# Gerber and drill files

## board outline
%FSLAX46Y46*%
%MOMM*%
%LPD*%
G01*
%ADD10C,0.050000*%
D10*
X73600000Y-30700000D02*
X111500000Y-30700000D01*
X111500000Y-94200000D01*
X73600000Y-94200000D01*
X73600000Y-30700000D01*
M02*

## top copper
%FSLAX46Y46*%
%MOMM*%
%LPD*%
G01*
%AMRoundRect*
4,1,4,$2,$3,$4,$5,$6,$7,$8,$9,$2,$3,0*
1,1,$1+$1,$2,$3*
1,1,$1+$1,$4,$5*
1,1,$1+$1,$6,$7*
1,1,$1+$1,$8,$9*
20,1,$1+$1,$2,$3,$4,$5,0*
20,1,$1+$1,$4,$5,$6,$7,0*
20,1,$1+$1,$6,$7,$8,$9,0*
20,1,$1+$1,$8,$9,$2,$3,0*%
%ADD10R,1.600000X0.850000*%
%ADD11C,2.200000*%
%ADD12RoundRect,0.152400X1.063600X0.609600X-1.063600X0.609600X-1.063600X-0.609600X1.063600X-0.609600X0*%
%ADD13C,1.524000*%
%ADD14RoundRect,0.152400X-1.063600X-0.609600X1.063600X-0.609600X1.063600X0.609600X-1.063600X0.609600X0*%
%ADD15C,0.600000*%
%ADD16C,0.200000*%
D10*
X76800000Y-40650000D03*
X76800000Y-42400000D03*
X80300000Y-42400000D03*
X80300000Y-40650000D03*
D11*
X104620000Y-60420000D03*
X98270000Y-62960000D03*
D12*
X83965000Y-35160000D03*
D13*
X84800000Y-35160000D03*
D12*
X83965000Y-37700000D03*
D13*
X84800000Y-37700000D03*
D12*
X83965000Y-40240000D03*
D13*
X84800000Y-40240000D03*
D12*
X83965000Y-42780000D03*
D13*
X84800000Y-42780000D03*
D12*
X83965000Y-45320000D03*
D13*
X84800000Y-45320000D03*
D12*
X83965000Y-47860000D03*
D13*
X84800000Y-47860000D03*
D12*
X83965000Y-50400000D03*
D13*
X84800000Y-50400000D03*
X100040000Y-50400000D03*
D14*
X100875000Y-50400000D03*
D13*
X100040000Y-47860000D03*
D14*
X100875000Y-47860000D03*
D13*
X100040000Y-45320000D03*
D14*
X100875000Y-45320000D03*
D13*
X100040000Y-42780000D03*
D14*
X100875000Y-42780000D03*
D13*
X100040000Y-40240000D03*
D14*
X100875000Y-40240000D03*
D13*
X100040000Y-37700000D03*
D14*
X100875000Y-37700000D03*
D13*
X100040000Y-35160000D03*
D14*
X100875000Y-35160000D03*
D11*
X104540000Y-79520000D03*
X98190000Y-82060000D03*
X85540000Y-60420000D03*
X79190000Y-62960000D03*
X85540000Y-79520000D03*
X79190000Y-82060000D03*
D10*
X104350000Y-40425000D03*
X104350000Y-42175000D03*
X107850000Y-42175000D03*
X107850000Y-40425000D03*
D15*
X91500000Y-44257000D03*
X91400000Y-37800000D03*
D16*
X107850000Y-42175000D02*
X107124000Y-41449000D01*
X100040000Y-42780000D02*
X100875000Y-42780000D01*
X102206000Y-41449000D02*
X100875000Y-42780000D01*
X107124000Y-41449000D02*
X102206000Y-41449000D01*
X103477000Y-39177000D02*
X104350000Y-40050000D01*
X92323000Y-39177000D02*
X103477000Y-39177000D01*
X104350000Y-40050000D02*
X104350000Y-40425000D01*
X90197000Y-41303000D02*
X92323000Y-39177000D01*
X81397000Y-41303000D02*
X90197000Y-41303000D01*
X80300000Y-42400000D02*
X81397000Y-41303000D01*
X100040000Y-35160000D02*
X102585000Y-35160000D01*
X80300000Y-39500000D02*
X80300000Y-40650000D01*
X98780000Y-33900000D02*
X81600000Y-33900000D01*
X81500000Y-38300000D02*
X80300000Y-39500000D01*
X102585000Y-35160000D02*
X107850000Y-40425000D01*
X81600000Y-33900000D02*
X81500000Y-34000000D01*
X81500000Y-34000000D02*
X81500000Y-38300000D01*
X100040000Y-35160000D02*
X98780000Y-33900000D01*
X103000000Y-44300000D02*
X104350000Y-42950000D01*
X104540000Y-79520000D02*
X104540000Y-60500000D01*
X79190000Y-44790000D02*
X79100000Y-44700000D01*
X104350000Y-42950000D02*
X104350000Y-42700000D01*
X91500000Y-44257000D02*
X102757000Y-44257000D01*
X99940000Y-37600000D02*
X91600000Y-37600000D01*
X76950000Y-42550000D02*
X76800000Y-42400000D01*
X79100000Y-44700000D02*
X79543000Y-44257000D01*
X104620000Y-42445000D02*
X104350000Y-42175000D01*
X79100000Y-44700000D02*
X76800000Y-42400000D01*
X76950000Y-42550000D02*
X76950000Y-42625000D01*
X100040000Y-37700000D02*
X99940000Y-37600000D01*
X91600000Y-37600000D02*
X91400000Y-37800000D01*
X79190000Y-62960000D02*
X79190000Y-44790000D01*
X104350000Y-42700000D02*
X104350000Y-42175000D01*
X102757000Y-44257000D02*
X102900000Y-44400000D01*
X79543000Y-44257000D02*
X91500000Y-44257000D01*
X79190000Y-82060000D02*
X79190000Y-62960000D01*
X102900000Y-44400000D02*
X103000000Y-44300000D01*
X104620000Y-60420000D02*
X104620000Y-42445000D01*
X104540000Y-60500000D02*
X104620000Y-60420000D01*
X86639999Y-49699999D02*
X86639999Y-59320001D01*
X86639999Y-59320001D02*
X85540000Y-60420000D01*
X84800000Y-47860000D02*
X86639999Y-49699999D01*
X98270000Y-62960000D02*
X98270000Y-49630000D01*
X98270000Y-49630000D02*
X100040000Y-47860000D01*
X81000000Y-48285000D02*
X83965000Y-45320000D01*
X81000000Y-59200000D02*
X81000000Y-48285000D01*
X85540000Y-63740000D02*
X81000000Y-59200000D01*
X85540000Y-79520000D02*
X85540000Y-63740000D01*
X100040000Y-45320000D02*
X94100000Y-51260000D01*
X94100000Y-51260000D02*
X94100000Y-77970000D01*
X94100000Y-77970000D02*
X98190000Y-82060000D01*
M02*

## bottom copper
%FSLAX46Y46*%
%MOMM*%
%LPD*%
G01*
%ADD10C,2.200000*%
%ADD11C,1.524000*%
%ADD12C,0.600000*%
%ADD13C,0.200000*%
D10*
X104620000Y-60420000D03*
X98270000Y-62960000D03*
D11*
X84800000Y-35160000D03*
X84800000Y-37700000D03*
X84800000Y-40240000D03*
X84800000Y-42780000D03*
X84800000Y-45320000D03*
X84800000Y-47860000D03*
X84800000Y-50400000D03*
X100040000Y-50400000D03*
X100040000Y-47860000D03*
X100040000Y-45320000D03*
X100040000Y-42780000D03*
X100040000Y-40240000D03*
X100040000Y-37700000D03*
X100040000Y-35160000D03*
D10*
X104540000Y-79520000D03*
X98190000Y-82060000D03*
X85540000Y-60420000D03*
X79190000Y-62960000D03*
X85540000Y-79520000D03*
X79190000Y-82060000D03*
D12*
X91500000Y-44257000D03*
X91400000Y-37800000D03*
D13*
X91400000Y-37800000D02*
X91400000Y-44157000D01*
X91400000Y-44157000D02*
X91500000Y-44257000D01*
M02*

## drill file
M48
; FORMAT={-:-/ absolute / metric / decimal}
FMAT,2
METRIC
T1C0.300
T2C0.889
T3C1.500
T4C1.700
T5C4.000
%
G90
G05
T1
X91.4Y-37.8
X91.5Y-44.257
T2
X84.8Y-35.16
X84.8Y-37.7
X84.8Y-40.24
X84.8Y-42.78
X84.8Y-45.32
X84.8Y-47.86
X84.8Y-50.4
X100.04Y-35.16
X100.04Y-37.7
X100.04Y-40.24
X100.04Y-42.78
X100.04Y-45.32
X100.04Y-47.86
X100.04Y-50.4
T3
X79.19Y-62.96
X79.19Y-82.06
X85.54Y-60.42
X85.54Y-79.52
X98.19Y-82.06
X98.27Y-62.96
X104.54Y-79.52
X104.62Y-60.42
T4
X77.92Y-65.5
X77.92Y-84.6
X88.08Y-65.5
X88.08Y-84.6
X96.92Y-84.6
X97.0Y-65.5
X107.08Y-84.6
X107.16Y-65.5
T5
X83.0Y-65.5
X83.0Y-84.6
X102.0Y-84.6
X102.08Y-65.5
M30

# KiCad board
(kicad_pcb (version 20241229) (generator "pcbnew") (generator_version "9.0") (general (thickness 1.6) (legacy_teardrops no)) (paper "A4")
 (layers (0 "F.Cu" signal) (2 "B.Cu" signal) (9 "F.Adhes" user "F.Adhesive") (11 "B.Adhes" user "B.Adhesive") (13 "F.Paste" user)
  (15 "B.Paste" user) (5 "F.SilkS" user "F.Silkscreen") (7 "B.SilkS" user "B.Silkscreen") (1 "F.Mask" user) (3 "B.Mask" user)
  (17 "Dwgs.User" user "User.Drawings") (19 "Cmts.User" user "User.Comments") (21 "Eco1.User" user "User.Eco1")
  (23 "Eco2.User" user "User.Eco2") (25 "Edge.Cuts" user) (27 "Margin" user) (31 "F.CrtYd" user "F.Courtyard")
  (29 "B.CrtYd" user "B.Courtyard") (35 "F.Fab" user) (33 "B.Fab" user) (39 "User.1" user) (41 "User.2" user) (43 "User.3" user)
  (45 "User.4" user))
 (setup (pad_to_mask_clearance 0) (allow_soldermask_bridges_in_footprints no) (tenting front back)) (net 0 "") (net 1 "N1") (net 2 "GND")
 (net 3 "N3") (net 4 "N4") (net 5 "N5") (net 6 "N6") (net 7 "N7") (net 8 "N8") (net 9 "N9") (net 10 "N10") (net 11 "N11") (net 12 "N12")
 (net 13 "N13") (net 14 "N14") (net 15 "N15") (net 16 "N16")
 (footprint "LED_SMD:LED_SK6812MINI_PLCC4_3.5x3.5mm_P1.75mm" (layer "F.Cu") (at 78.55 41.525)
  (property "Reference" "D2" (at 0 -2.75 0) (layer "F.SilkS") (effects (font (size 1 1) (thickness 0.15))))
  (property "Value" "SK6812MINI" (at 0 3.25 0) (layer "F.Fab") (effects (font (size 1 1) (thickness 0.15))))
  (pad "1" smd rect (at -1.75 -0.875) (size 1.6 0.85) (layers "F.Cu" "F.Mask" "F.Paste") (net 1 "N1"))
  (pad "2" smd rect (at -1.75 0.875) (size 1.6 0.85) (layers "F.Cu" "F.Mask" "F.Paste") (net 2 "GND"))
  (pad "3" smd rect (at 1.75 0.875) (size 1.6 0.85) (layers "F.Cu" "F.Mask" "F.Paste") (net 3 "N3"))
  (pad "4" smd rect (at 1.75 -0.875) (size 1.6 0.85) (layers "F.Cu" "F.Mask" "F.Paste") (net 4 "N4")))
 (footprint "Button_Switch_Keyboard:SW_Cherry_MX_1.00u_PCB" (layer "F.Cu") (at 104.62 60.42)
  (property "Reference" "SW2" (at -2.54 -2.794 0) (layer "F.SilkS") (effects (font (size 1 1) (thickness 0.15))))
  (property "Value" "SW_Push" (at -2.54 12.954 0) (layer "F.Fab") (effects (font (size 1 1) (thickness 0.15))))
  (pad "" np_thru_hole circle (at -7.62 5.08) (size 1.7 1.7) (drill 1.7) (layers "*.Cu" "*.Mask"))
  (pad "" np_thru_hole circle (at -2.54 5.08) (size 4 4) (drill 4) (layers "*.Cu" "*.Mask"))
  (pad "" np_thru_hole circle (at 2.54 5.08) (size 1.7 1.7) (drill 1.7) (layers "*.Cu" "*.Mask"))
  (pad "1" thru_hole circle (at 0 0) (size 2.2 2.2) (drill 1.5) (layers "*.Cu" "*.Mask") (remove_unused_layers no) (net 2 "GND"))
  (pad "2" thru_hole circle (at -6.35 2.54) (size 2.2 2.2) (drill 1.5) (layers "*.Cu" "*.Mask") (remove_unused_layers no) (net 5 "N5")))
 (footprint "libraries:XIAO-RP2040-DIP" (layer "F.Cu") (at 92.42 42.78)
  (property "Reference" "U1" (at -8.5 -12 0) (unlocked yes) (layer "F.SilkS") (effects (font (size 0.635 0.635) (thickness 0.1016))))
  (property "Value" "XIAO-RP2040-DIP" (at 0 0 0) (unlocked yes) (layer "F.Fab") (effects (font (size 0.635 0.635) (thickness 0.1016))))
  (pad "1" smd roundrect (at -8.455 -7.62 180) (size 2.432 1.524) (layers "F.Cu" "F.Mask") (roundrect_rratio 0.1) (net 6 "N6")
   (thermal_bridge_angle 45))
  (pad "1" thru_hole circle (at -7.62 -7.62 180) (size 1.524 1.524) (drill 0.889) (layers "*.Cu" "*.Mask") (remove_unused_layers no)
   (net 6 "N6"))
  (pad "2" smd roundrect (at -8.455 -5.08 180) (size 2.432 1.524) (layers "F.Cu" "F.Mask") (roundrect_rratio 0.1) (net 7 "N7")
   (thermal_bridge_angle 45))
  (pad "2" thru_hole circle (at -7.62 -5.08 180) (size 1.524 1.524) (drill 0.889) (layers "*.Cu" "*.Mask") (remove_unused_layers no)
   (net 7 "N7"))
  (pad "3" smd roundrect (at -8.455 -2.54 180) (size 2.432 1.524) (layers "F.Cu" "F.Mask") (roundrect_rratio 0.1) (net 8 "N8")
   (thermal_bridge_angle 45))
  (pad "3" thru_hole circle (at -7.62 -2.54 180) (size 1.524 1.524) (drill 0.889) (layers "*.Cu" "*.Mask") (remove_unused_layers no)
   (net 8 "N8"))
  (pad "4" smd roundrect (at -8.455 0 180) (size 2.432 1.524) (layers "F.Cu" "F.Mask") (roundrect_rratio 0.1) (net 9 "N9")
   (thermal_bridge_angle 45))
  (pad "4" thru_hole circle (at -7.62 0 180) (size 1.524 1.524) (drill 0.889) (layers "*.Cu" "*.Mask") (remove_unused_layers no)
   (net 9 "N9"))
  (pad "5" smd roundrect (at -8.455 2.54 180) (size 2.432 1.524) (layers "F.Cu" "F.Mask") (roundrect_rratio 0.1) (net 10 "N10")
   (thermal_bridge_angle 45))
  (pad "5" thru_hole circle (at -7.62 2.54 180) (size 1.524 1.524) (drill 0.889) (layers "*.Cu" "*.Mask") (remove_unused_layers no)
   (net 10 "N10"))
  (pad "6" smd roundrect (at -8.455 5.08 180) (size 2.432 1.524) (layers "F.Cu" "F.Mask") (roundrect_rratio 0.1) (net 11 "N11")
   (thermal_bridge_angle 45))
  (pad "6" thru_hole circle (at -7.62 5.08 180) (size 1.524 1.524) (drill 0.889) (layers "*.Cu" "*.Mask") (remove_unused_layers no)
   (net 11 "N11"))
  (pad "7" smd roundrect (at -8.455 7.62 180) (size 2.432 1.524) (layers "F.Cu" "F.Mask") (roundrect_rratio 0.1) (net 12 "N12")
   (thermal_bridge_angle 45))
  (pad "7" thru_hole circle (at -7.62 7.62 180) (size 1.524 1.524) (drill 0.889) (layers "*.Cu" "*.Mask") (remove_unused_layers no)
   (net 12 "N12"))
  (pad "8" thru_hole circle (at 7.62 7.62) (size 1.524 1.524) (drill 0.889) (layers "*.Cu" "*.Mask") (remove_unused_layers no)
   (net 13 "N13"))
  (pad "8" smd roundrect (at 8.455 7.62) (size 2.432 1.524) (layers "F.Cu" "F.Mask") (roundrect_rratio 0.1) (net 13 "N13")
   (thermal_bridge_angle 45))
  (pad "9" thru_hole circle (at 7.62 5.08) (size 1.524 1.524) (drill 0.889) (layers "*.Cu" "*.Mask") (remove_unused_layers no) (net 5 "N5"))
  (pad "9" smd roundrect (at 8.455 5.08) (size 2.432 1.524) (layers "F.Cu" "F.Mask") (roundrect_rratio 0.1) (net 5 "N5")
   (thermal_bridge_angle 45))
  (pad "10" thru_hole circle (at 7.62 2.54) (size 1.524 1.524) (drill 0.889) (layers "*.Cu" "*.Mask") (remove_unused_layers no)
   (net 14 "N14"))
  (pad "10" smd roundrect (at 8.455 2.54) (size 2.432 1.524) (layers "F.Cu" "F.Mask") (roundrect_rratio 0.1) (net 14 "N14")
   (thermal_bridge_angle 45))
  (pad "11" thru_hole circle (at 7.62 0) (size 1.524 1.524) (drill 0.889) (layers "*.Cu" "*.Mask") (remove_unused_layers no) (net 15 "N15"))
  (pad "11" smd roundrect (at 8.455 0) (size 2.432 1.524) (layers "F.Cu" "F.Mask") (roundrect_rratio 0.1) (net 15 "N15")
   (thermal_bridge_angle 45))
  (pad "12" thru_hole circle (at 7.62 -2.54) (size 1.524 1.524) (drill 0.889) (layers "*.Cu" "*.Mask") (remove_unused_layers no)
   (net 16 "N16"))
  (pad "12" smd roundrect (at 8.455 -2.54) (size 2.432 1.524) (layers "F.Cu" "F.Mask") (roundrect_rratio 0.1) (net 16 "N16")
   (thermal_bridge_angle 45))
  (pad "13" thru_hole circle (at 7.62 -5.08) (size 1.524 1.524) (drill 0.889) (layers "*.Cu" "*.Mask") (remove_unused_layers no)
   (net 2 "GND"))
  (pad "13" smd roundrect (at 8.455 -5.08) (size 2.432 1.524) (layers "F.Cu" "F.Mask") (roundrect_rratio 0.1) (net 2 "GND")
   (thermal_bridge_angle 45))
  (pad "14" thru_hole circle (at 7.62 -7.62) (size 1.524 1.524) (drill 0.889) (layers "*.Cu" "*.Mask") (remove_unused_layers no)
   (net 4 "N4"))
  (pad "14" smd roundrect (at 8.455 -7.62) (size 2.432 1.524) (layers "F.Cu" "F.Mask") (roundrect_rratio 0.1) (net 4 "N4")
   (thermal_bridge_angle 45)))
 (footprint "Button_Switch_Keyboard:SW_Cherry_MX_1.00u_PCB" (layer "F.Cu") (at 104.54 79.52)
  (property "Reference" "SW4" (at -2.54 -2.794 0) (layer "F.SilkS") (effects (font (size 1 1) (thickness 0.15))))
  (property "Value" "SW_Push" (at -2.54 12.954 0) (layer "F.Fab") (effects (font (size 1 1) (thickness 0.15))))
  (pad "" np_thru_hole circle (at -7.62 5.08) (size 1.7 1.7) (drill 1.7) (layers "*.Cu" "*.Mask"))
  (pad "" np_thru_hole circle (at -2.54 5.08) (size 4 4) (drill 4) (layers "*.Cu" "*.Mask"))
  (pad "" np_thru_hole circle (at 2.54 5.08) (size 1.7 1.7) (drill 1.7) (layers "*.Cu" "*.Mask"))
  (pad "1" thru_hole circle (at 0 0) (size 2.2 2.2) (drill 1.5) (layers "*.Cu" "*.Mask") (remove_unused_layers no) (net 2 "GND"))
  (pad "2" thru_hole circle (at -6.35 2.54) (size 2.2 2.2) (drill 1.5) (layers "*.Cu" "*.Mask") (remove_unused_layers no) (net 14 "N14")))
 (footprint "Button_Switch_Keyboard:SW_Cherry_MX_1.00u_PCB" (layer "F.Cu") (at 85.54 60.42)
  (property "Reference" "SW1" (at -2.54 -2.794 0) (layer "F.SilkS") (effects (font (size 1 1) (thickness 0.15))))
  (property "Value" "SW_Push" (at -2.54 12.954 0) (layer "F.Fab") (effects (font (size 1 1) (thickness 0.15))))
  (pad "" np_thru_hole circle (at -7.62 5.08) (size 1.7 1.7) (drill 1.7) (layers "*.Cu" "*.Mask"))
  (pad "" np_thru_hole circle (at -2.54 5.08) (size 4 4) (drill 4) (layers "*.Cu" "*.Mask"))
  (pad "" np_thru_hole circle (at 2.54 5.08) (size 1.7 1.7) (drill 1.7) (layers "*.Cu" "*.Mask"))
  (pad "1" thru_hole circle (at 0 0) (size 2.2 2.2) (drill 1.5) (layers "*.Cu" "*.Mask") (remove_unused_layers no) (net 11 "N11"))
  (pad "2" thru_hole circle (at -6.35 2.54) (size 2.2 2.2) (drill 1.5) (layers "*.Cu" "*.Mask") (remove_unused_layers no) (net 2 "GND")))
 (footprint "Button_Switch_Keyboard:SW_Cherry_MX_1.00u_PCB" (layer "F.Cu") (at 85.54 79.52)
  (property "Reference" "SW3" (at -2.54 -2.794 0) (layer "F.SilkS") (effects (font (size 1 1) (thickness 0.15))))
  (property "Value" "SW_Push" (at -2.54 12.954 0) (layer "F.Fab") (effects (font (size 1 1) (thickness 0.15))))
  (pad "" np_thru_hole circle (at -7.62 5.08) (size 1.7 1.7) (drill 1.7) (layers "*.Cu" "*.Mask"))
  (pad "" np_thru_hole circle (at -2.54 5.08) (size 4 4) (drill 4) (layers "*.Cu" "*.Mask"))
  (pad "" np_thru_hole circle (at 2.54 5.08) (size 1.7 1.7) (drill 1.7) (layers "*.Cu" "*.Mask"))
  (pad "1" thru_hole circle (at 0 0) (size 2.2 2.2) (drill 1.5) (layers "*.Cu" "*.Mask") (remove_unused_layers no) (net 10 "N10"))
  (pad "2" thru_hole circle (at -6.35 2.54) (size 2.2 2.2) (drill 1.5) (layers "*.Cu" "*.Mask") (remove_unused_layers no) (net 2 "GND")))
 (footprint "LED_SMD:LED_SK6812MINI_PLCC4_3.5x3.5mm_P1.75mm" (layer "F.Cu") (at 106.1 41.3)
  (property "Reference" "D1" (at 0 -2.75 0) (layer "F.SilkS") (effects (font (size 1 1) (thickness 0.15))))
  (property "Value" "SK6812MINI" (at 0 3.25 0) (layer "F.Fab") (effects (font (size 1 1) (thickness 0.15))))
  (pad "1" smd rect (at -1.75 -0.875) (size 1.6 0.85) (layers "F.Cu" "F.Mask" "F.Paste") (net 3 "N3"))
  (pad "2" smd rect (at -1.75 0.875) (size 1.6 0.85) (layers "F.Cu" "F.Mask" "F.Paste") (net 2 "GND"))
  (pad "3" smd rect (at 1.75 0.875) (size 1.6 0.85) (layers "F.Cu" "F.Mask" "F.Paste") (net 15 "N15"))
  (pad "4" smd rect (at 1.75 -0.875) (size 1.6 0.85) (layers "F.Cu" "F.Mask" "F.Paste") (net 4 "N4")))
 (gr_rect (start 73.6 30.7) (end 111.5 94.2) (stroke (width 0.05) (type default)) (fill no) (layer "Edge.Cuts"))
 (segment (start 107.85 42.175) (end 107.124 41.449) (width 0.2) (layer "F.Cu") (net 15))
 (segment (start 100.04 42.78) (end 100.875 42.78) (width 0.2) (layer "F.Cu") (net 15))
 (segment (start 102.206 41.449) (end 100.875 42.78) (width 0.2) (layer "F.Cu") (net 15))
 (segment (start 107.124 41.449) (end 102.206 41.449) (width 0.2) (layer "F.Cu") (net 15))
 (segment (start 103.477 39.177) (end 104.35 40.05) (width 0.2) (layer "F.Cu") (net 3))
 (segment (start 92.323 39.177) (end 103.477 39.177) (width 0.2) (layer "F.Cu") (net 3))
 (segment (start 104.35 40.05) (end 104.35 40.425) (width 0.2) (layer "F.Cu") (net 3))
 (segment (start 90.197 41.303) (end 92.323 39.177) (width 0.2) (layer "F.Cu") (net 3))
 (segment (start 81.397 41.303) (end 90.197 41.303) (width 0.2) (layer "F.Cu") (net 3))
 (segment (start 80.3 42.4) (end 81.397 41.303) (width 0.2) (layer "F.Cu") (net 3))
 (segment (start 100.04 35.16) (end 102.585 35.16) (width 0.2) (layer "F.Cu") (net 4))
 (segment (start 80.3 39.5) (end 80.3 40.65) (width 0.2) (layer "F.Cu") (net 4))
 (segment (start 98.78 33.9) (end 81.6 33.9) (width 0.2) (layer "F.Cu") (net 4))
 (segment (start 81.5 38.3) (end 80.3 39.5) (width 0.2) (layer "F.Cu") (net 4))
 (segment (start 102.585 35.16) (end 107.85 40.425) (width 0.2) (layer "F.Cu") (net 4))
 (segment (start 81.6 33.9) (end 81.5 34) (width 0.2) (layer "F.Cu") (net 4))
 (segment (start 81.5 34) (end 81.5 38.3) (width 0.2) (layer "F.Cu") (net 4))
 (segment (start 100.04 35.16) (end 98.78 33.9) (width 0.2) (layer "F.Cu") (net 4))
 (segment (start 103 44.3) (end 104.35 42.95) (width 0.2) (layer "F.Cu") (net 2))
 (segment (start 104.54 79.52) (end 104.54 60.5) (width 0.2) (layer "F.Cu") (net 2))
 (segment (start 79.19 44.79) (end 79.1 44.7) (width 0.2) (layer "F.Cu") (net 2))
 (segment (start 104.35 42.95) (end 104.35 42.7) (width 0.2) (layer "F.Cu") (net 2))
 (segment (start 91.5 44.257) (end 102.757 44.257) (width 0.2) (layer "F.Cu") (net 2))
 (segment (start 99.94 37.6) (end 91.6 37.6) (width 0.2) (layer "F.Cu") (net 2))
 (segment (start 76.95 42.55) (end 76.8 42.4) (width 0.2) (layer "F.Cu") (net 2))
 (segment (start 79.1 44.7) (end 79.543 44.257) (width 0.2) (layer "F.Cu") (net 2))
 (segment (start 104.62 42.445) (end 104.35 42.175) (width 0.2) (layer "F.Cu") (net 2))
 (segment (start 79.1 44.7) (end 76.8 42.4) (width 0.2) (layer "F.Cu") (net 2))
 (segment (start 76.95 42.55) (end 76.95 42.625) (width 0.2) (layer "F.Cu") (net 2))
 (segment (start 100.04 37.7) (end 99.94 37.6) (width 0.2) (layer "F.Cu") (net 2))
 (segment (start 91.6 37.6) (end 91.4 37.8) (width 0.2) (layer "F.Cu") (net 2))
 (segment (start 79.19 62.96) (end 79.19 44.79) (width 0.2) (layer "F.Cu") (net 2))
 (segment (start 104.35 42.7) (end 104.35 42.175) (width 0.2) (layer "F.Cu") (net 2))
 (segment (start 102.757 44.257) (end 102.9 44.4) (width 0.2) (layer "F.Cu") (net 2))
 (segment (start 79.543 44.257) (end 91.5 44.257) (width 0.2) (layer "F.Cu") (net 2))
 (segment (start 79.19 82.06) (end 79.19 62.96) (width 0.2) (layer "F.Cu") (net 2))
 (segment (start 102.9 44.4) (end 103 44.3) (width 0.2) (layer "F.Cu") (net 2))
 (segment (start 104.62 60.42) (end 104.62 42.445) (width 0.2) (layer "F.Cu") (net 2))
 (segment (start 104.54 60.5) (end 104.62 60.42) (width 0.2) (layer "F.Cu") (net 2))
 (via (at 91.5 44.257) (size 0.6) (drill 0.3) (layers "F.Cu" "B.Cu") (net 2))
 (via (at 91.4 37.8) (size 0.6) (drill 0.3) (layers "F.Cu" "B.Cu") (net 2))
 (segment (start 91.4 37.8) (end 91.4 44.157) (width 0.2) (layer "B.Cu") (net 2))
 (segment (start 91.4 44.157) (end 91.5 44.257) (width 0.2) (layer "B.Cu") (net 2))
 (segment (start 86.639999 49.699999) (end 86.639999 59.320001) (width 0.2) (layer "F.Cu") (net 11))
 (segment (start 86.639999 59.320001) (end 85.54 60.42) (width 0.2) (layer "F.Cu") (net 11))
 (segment (start 84.8 47.86) (end 86.639999 49.699999) (width 0.2) (layer "F.Cu") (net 11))
 (segment (start 98.27 62.96) (end 98.27 49.63) (width 0.2) (layer "F.Cu") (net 5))
 (segment (start 98.27 49.63) (end 100.04 47.86) (width 0.2) (layer "F.Cu") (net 5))
 (segment (start 81 48.285) (end 83.965 45.32) (width 0.2) (layer "F.Cu") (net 10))
 (segment (start 81 59.2) (end 81 48.285) (width 0.2) (layer "F.Cu") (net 10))
 (segment (start 85.54 63.74) (end 81 59.2) (width 0.2) (layer "F.Cu") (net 10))
 (segment (start 85.54 79.52) (end 85.54 63.74) (width 0.2) (layer "F.Cu") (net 10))
 (segment (start 100.04 45.32) (end 94.1 51.26) (width 0.2) (layer "F.Cu") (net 14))
 (segment (start 94.1 51.26) (end 94.1 77.97) (width 0.2) (layer "F.Cu") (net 14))
 (segment (start 94.1 77.97) (end 98.19 82.06) (width 0.2) (layer "F.Cu") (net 14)))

